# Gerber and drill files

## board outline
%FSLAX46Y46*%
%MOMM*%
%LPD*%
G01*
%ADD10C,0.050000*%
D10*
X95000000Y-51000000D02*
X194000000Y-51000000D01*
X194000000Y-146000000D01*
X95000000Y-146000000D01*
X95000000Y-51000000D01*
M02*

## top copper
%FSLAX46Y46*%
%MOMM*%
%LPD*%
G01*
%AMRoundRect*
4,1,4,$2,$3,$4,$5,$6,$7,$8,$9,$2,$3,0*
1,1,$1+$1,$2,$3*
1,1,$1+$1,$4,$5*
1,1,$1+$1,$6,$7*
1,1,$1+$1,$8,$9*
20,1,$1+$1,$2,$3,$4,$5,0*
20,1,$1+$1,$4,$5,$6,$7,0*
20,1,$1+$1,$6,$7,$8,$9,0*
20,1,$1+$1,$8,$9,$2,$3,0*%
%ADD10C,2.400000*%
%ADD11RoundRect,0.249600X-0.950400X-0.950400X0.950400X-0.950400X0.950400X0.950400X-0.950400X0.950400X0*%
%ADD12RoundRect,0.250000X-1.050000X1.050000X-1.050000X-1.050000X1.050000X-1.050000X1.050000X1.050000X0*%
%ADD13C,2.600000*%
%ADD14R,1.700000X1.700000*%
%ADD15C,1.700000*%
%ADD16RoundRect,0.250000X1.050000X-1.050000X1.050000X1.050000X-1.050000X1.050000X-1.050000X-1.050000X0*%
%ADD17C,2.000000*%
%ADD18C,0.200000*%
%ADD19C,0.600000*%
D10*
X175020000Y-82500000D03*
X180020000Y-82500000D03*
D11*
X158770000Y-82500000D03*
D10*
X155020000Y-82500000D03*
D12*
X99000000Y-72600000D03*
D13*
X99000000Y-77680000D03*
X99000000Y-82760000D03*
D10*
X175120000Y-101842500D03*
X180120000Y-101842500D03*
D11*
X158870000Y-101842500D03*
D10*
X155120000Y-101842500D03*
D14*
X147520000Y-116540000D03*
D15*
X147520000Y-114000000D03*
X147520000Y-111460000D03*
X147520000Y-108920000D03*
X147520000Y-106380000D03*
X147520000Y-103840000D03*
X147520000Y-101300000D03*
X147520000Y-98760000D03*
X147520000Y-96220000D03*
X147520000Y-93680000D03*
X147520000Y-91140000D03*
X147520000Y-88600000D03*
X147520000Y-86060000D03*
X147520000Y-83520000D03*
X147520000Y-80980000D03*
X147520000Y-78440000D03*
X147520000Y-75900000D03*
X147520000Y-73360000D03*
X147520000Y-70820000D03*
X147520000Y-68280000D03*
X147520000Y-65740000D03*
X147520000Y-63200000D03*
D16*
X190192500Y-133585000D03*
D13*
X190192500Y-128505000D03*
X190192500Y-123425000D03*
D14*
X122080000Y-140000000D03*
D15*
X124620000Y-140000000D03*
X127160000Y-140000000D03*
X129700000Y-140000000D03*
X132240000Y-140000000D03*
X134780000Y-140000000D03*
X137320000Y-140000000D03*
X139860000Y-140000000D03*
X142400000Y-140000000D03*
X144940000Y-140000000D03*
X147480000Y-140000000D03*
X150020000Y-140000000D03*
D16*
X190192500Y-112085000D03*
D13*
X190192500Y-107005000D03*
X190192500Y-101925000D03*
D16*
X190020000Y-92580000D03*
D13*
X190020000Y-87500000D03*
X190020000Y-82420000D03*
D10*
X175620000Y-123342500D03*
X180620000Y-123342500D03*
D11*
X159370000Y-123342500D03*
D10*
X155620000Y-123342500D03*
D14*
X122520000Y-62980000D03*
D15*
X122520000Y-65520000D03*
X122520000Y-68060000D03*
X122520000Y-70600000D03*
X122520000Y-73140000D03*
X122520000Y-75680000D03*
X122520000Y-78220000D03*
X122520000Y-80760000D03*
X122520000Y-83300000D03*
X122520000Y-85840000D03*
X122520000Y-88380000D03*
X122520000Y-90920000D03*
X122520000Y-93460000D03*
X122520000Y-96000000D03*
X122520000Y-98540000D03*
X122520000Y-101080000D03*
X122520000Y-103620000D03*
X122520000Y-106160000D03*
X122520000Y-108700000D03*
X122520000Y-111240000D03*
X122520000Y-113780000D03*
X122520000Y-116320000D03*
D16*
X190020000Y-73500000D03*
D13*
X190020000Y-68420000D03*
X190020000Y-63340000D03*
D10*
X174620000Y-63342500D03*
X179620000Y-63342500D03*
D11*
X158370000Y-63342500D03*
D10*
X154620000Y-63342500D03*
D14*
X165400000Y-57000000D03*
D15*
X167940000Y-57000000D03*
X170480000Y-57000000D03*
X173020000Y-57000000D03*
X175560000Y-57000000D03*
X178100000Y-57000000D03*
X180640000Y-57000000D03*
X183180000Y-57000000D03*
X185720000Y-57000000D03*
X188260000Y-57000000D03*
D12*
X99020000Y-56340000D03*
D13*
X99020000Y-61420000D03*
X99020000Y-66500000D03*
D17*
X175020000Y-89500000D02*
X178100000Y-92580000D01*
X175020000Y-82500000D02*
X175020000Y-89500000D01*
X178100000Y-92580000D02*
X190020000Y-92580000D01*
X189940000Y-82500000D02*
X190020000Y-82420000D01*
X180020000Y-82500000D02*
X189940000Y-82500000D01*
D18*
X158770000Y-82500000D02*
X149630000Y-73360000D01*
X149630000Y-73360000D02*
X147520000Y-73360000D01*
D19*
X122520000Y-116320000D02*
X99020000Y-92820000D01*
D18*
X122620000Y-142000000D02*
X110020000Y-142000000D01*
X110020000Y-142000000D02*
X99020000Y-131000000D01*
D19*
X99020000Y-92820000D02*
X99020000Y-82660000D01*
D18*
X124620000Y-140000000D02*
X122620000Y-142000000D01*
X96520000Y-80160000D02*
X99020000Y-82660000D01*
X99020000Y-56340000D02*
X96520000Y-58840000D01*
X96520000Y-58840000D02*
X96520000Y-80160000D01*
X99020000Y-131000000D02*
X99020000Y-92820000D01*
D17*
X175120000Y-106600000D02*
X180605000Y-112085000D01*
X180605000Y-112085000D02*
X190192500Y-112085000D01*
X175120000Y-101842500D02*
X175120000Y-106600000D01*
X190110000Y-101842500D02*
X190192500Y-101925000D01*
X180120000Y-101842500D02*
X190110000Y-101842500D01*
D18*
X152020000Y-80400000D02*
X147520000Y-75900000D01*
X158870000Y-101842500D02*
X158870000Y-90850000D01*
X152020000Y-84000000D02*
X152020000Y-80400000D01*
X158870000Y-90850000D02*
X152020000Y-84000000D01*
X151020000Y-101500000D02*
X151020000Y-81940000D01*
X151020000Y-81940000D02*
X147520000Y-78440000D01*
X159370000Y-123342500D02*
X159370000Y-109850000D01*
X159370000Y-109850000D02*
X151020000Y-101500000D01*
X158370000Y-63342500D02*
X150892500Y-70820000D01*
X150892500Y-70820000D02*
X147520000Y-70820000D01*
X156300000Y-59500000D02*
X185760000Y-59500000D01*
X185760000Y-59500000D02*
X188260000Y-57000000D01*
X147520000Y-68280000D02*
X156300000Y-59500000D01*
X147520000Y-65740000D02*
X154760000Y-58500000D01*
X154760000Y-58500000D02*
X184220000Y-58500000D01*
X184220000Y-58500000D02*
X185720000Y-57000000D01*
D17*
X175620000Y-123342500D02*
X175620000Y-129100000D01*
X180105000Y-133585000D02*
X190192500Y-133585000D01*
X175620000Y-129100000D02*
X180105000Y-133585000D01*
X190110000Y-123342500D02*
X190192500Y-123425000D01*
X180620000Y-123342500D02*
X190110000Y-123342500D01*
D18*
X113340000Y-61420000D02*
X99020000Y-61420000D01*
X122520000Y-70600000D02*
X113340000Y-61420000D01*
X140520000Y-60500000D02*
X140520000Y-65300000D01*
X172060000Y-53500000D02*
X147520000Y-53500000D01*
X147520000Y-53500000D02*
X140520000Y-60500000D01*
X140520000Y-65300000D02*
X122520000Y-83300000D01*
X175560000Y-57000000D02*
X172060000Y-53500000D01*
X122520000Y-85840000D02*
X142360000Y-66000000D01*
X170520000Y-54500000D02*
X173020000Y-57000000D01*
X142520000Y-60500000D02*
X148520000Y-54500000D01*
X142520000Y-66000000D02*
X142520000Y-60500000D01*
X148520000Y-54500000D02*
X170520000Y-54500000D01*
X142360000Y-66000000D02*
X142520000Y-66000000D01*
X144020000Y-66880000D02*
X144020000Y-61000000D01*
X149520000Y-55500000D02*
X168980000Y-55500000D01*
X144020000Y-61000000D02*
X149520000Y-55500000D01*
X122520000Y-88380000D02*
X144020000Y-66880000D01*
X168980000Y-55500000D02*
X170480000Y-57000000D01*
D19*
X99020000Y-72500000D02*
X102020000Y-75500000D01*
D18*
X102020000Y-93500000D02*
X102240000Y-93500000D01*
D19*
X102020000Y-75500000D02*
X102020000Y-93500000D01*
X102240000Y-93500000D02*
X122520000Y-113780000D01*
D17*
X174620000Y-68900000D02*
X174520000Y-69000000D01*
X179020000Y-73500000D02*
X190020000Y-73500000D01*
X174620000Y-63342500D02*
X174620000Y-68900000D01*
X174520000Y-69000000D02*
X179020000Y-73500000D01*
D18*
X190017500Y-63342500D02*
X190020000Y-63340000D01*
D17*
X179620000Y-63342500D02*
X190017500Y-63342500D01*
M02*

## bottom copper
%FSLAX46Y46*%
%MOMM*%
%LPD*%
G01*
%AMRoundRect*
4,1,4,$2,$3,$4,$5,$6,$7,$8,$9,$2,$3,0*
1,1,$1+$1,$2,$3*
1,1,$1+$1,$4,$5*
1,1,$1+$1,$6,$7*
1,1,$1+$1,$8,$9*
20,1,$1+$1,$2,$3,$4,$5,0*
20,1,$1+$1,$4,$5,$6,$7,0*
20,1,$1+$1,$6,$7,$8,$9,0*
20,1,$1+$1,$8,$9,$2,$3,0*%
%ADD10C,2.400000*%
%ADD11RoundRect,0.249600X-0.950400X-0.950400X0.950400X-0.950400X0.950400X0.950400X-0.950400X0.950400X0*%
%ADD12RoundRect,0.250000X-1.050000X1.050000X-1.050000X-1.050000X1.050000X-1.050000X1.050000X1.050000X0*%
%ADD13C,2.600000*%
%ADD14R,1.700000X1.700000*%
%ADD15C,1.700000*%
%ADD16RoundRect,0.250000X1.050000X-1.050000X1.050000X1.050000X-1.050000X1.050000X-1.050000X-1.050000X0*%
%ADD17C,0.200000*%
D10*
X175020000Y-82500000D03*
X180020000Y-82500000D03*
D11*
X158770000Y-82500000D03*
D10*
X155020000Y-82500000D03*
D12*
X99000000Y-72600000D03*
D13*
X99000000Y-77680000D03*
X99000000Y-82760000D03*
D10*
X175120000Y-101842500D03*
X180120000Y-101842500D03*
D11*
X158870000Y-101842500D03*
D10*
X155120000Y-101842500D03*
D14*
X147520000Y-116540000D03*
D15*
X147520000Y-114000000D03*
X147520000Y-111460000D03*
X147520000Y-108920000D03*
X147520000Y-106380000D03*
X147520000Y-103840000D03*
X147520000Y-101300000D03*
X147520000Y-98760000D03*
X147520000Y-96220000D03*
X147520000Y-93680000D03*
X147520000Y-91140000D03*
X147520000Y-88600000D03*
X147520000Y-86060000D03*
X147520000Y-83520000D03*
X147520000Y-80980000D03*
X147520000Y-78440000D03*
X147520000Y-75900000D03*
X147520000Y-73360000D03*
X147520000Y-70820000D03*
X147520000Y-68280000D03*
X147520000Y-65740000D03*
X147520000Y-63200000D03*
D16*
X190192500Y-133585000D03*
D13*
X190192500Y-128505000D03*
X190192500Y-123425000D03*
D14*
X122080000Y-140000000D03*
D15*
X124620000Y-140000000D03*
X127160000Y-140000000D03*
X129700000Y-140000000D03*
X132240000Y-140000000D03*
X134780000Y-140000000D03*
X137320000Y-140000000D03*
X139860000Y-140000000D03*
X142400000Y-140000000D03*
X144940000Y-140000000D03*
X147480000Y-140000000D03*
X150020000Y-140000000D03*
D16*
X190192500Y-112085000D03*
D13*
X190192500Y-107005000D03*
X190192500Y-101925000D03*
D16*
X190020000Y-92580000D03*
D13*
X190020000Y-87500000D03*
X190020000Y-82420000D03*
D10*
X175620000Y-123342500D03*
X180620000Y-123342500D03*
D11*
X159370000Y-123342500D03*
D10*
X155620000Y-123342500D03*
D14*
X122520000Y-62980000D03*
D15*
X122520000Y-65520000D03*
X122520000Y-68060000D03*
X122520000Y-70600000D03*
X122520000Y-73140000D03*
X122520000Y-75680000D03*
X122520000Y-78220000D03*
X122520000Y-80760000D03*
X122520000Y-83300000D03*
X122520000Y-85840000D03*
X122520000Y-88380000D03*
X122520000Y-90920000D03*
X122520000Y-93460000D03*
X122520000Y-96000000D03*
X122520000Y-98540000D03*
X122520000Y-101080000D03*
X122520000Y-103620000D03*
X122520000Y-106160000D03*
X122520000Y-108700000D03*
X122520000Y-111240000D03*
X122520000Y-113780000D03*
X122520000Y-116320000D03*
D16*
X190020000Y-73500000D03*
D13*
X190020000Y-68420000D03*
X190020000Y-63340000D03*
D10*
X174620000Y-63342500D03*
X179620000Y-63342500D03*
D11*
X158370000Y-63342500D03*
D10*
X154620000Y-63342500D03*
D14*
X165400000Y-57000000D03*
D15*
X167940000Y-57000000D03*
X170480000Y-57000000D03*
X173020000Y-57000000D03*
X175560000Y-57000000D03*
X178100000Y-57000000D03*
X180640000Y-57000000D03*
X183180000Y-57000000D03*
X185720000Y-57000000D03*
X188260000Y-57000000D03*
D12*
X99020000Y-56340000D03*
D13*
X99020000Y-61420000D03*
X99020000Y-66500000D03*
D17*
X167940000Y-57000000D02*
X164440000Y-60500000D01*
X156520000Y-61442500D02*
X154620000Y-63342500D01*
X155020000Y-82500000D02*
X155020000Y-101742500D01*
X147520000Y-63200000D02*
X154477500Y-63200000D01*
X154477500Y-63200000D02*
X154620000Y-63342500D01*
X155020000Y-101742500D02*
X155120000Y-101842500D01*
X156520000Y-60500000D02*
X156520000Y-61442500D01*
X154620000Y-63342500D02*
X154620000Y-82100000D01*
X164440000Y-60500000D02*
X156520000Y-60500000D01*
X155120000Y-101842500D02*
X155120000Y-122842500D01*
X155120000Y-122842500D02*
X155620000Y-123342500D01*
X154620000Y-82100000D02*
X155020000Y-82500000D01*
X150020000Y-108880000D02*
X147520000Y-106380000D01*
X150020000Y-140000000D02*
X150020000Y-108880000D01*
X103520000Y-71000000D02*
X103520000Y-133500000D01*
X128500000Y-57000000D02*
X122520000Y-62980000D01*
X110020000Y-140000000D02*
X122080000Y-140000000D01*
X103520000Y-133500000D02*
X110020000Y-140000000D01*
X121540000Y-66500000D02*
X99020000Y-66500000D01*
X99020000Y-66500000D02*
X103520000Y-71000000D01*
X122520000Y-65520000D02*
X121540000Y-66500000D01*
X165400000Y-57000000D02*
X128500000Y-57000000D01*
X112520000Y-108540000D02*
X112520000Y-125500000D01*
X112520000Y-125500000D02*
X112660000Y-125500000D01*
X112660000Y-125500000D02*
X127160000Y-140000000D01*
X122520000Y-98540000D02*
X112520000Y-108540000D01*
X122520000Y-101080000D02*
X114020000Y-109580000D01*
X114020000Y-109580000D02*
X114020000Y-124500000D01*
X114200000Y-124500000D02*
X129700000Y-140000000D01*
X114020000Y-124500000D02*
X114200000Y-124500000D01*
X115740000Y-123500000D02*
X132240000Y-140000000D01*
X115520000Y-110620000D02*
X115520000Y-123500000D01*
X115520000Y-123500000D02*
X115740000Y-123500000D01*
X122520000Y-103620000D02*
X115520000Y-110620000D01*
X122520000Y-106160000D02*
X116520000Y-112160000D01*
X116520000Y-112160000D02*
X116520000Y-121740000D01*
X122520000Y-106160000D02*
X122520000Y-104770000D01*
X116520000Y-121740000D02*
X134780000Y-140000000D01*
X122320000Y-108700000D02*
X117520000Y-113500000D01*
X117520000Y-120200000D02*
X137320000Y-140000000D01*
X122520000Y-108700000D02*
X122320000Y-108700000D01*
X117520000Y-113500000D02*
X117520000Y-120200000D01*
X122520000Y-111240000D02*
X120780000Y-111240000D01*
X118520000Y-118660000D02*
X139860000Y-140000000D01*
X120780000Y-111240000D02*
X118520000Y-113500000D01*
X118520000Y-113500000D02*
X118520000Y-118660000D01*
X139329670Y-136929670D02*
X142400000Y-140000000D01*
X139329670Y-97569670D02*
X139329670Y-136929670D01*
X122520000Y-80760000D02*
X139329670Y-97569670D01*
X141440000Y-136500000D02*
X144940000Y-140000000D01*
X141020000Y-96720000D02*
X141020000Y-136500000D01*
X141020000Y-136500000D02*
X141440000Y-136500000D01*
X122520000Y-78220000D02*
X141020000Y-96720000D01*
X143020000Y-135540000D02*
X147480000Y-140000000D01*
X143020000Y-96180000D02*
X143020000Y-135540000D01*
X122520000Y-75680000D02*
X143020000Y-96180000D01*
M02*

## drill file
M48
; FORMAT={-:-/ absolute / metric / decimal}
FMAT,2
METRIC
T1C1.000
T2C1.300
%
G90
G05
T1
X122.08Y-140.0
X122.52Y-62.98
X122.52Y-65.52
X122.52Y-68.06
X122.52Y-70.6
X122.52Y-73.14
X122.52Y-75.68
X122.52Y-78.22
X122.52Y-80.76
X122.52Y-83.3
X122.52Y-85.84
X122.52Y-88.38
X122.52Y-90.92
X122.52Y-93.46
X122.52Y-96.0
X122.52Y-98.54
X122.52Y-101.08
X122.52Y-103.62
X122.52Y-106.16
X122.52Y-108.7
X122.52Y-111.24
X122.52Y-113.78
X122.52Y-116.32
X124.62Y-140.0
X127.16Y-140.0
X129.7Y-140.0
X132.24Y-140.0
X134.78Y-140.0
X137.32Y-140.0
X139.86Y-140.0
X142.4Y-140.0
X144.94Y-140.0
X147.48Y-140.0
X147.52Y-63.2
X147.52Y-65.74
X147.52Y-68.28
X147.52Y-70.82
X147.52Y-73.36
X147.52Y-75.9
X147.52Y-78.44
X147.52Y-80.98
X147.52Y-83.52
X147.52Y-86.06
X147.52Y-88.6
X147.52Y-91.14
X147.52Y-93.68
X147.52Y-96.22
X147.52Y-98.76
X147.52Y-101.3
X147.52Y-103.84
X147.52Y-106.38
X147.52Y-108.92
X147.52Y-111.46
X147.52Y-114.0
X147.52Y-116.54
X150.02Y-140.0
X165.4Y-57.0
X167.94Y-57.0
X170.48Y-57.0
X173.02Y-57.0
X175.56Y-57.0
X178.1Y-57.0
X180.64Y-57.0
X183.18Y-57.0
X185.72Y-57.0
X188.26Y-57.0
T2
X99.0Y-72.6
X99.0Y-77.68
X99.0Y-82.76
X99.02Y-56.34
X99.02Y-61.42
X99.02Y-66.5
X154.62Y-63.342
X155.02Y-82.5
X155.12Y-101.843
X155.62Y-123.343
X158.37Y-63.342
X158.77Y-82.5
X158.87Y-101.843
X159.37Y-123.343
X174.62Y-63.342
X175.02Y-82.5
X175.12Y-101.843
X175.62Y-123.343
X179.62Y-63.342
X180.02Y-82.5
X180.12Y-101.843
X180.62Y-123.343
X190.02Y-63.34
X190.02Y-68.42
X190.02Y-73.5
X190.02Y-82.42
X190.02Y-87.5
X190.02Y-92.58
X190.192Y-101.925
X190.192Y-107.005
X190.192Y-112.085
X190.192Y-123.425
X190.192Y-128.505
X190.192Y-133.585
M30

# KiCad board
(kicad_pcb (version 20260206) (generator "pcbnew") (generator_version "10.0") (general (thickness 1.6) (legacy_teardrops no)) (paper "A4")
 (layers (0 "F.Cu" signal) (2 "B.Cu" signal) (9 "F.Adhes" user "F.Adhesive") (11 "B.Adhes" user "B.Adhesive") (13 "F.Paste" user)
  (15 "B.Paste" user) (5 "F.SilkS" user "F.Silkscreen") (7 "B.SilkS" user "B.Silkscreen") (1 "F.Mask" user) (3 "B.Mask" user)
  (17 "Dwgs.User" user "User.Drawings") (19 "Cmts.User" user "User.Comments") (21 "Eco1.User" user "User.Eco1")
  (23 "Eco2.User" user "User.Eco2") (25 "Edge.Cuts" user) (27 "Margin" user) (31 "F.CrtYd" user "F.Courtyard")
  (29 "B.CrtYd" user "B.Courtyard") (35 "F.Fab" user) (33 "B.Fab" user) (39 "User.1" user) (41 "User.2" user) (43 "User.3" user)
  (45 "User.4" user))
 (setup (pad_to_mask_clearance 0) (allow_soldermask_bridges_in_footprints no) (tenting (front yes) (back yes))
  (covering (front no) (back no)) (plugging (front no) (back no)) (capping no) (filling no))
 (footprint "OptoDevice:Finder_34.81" (layer "F.Cu") (at 158.77 82.5)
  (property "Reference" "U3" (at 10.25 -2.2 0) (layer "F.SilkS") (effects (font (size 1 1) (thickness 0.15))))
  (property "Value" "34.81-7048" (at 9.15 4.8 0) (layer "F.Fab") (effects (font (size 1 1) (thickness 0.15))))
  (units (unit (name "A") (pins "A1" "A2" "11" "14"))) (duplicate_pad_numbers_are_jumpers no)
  (pad "11" thru_hole circle (at 16.25 0) (size 2.4 2.4) (drill 1.3) (layers "*.Cu" "*.Mask") (remove_unused_layers no)
   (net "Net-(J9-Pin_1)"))
  (pad "14" thru_hole circle (at 21.25 0) (size 2.4 2.4) (drill 1.3) (layers "*.Cu" "*.Mask") (remove_unused_layers no)
   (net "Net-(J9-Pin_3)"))
  (pad "A1" thru_hole roundrect (at 0 0) (size 2.4 2.4) (drill 1.3) (layers "*.Cu" "*.Mask") (remove_unused_layers no)
   (roundrect_rratio 0.104) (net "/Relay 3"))
  (pad "A2" thru_hole circle (at -3.75 0) (size 2.4 2.4) (drill 1.3) (layers "*.Cu" "*.Mask") (remove_unused_layers no) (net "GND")))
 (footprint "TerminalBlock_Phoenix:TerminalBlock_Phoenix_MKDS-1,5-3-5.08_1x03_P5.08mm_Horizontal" (layer "F.Cu") (at 99 72.6 -90)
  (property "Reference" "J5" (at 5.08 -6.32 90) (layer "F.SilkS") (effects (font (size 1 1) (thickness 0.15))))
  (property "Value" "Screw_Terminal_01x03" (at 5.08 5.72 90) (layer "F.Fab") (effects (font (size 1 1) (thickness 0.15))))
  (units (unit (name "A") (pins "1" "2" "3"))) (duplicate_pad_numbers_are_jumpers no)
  (pad "1" thru_hole roundrect (at 0 0 270) (size 2.6 2.6) (drill 1.3) (layers "*.Cu" "*.Mask") (remove_unused_layers no)
   (roundrect_rratio 0.096154) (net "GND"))
  (pad "2" thru_hole circle (at 5.08 0 270) (size 2.6 2.6) (drill 1.3) (layers "*.Cu" "*.Mask") (remove_unused_layers no)
   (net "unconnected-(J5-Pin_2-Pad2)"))
  (pad "3" thru_hole circle (at 10.16 0 270) (size 2.6 2.6) (drill 1.3) (layers "*.Cu" "*.Mask") (remove_unused_layers no) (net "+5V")))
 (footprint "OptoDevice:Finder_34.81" (layer "F.Cu") (at 158.87 101.8425)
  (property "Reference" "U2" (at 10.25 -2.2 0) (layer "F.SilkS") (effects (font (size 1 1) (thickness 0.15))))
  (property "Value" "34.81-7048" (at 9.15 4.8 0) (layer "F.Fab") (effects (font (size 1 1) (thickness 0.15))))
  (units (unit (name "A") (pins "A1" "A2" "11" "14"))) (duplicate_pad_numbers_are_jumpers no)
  (pad "11" thru_hole circle (at 16.25 0) (size 2.4 2.4) (drill 1.3) (layers "*.Cu" "*.Mask") (remove_unused_layers no)
   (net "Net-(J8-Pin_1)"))
  (pad "14" thru_hole circle (at 21.25 0) (size 2.4 2.4) (drill 1.3) (layers "*.Cu" "*.Mask") (remove_unused_layers no)
   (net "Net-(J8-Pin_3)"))
  (pad "A1" thru_hole roundrect (at 0 0) (size 2.4 2.4) (drill 1.3) (layers "*.Cu" "*.Mask") (remove_unused_layers no)
   (roundrect_rratio 0.104) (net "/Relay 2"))
  (pad "A2" thru_hole circle (at -3.75 0) (size 2.4 2.4) (drill 1.3) (layers "*.Cu" "*.Mask") (remove_unused_layers no) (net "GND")))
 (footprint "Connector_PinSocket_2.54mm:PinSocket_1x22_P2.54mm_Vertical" (layer "F.Cu") (at 147.52 116.54 180)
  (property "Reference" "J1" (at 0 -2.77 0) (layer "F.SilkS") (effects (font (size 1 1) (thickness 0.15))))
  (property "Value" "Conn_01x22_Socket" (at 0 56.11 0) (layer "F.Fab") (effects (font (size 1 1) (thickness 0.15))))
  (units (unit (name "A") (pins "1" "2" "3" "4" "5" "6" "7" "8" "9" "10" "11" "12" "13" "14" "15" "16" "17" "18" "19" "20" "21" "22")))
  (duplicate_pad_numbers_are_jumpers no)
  (pad "1" thru_hole rect (at 0 0 180) (size 1.7 1.7) (drill 1) (layers "*.Cu" "*.Mask") (remove_unused_layers no) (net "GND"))
  (pad "2" thru_hole circle (at 0 2.54 180) (size 1.7 1.7) (drill 1) (layers "*.Cu" "*.Mask") (remove_unused_layers no) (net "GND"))
  (pad "3" thru_hole circle (at 0 5.08 180) (size 1.7 1.7) (drill 1) (layers "*.Cu" "*.Mask") (remove_unused_layers no)
   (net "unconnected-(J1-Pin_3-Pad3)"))
  (pad "4" thru_hole circle (at 0 7.62 180) (size 1.7 1.7) (drill 1) (layers "*.Cu" "*.Mask") (remove_unused_layers no)
   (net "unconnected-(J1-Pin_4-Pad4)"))
  (pad "5" thru_hole circle (at 0 10.16 180) (size 1.7 1.7) (drill 1) (layers "*.Cu" "*.Mask") (remove_unused_layers no) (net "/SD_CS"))
  (pad "6" thru_hole circle (at 0 12.7 180) (size 1.7 1.7) (drill 1) (layers "*.Cu" "*.Mask") (remove_unused_layers no)
   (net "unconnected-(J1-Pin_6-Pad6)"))
  (pad "7" thru_hole circle (at 0 15.24 180) (size 1.7 1.7) (drill 1) (layers "*.Cu" "*.Mask") (remove_unused_layers no)
   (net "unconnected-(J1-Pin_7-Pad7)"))
  (pad "8" thru_hole circle (at 0 17.78 180) (size 1.7 1.7) (drill 1) (layers "*.Cu" "*.Mask") (remove_unused_layers no)
   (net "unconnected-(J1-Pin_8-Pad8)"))
  (pad "9" thru_hole circle (at 0 20.32 180) (size 1.7 1.7) (drill 1) (layers "*.Cu" "*.Mask") (remove_unused_layers no)
   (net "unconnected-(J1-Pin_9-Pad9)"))
  (pad "10" thru_hole circle (at 0 22.86 180) (size 1.7 1.7) (drill 1) (layers "*.Cu" "*.Mask") (remove_unused_layers no)
   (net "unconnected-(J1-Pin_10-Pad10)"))
  (pad "11" thru_hole circle (at 0 25.4 180) (size 1.7 1.7) (drill 1) (layers "*.Cu" "*.Mask") (remove_unused_layers no)
   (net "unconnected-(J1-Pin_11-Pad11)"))
  (pad "12" thru_hole circle (at 0 27.94 180) (size 1.7 1.7) (drill 1) (layers "*.Cu" "*.Mask") (remove_unused_layers no)
   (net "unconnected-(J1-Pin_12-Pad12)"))
  (pad "13" thru_hole circle (at 0 30.48 180) (size 1.7 1.7) (drill 1) (layers "*.Cu" "*.Mask") (remove_unused_layers no)
   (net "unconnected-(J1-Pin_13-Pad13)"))
  (pad "14" thru_hole circle (at 0 33.02 180) (size 1.7 1.7) (drill 1) (layers "*.Cu" "*.Mask") (remove_unused_layers no)
   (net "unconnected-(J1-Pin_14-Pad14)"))
  (pad "15" thru_hole circle (at 0 35.56 180) (size 1.7 1.7) (drill 1) (layers "*.Cu" "*.Mask") (remove_unused_layers no)
   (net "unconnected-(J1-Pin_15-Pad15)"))
  (pad "16" thru_hole circle (at 0 38.1 180) (size 1.7 1.7) (drill 1) (layers "*.Cu" "*.Mask") (remove_unused_layers no) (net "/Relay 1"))
  (pad "17" thru_hole circle (at 0 40.64 180) (size 1.7 1.7) (drill 1) (layers "*.Cu" "*.Mask") (remove_unused_layers no) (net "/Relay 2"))
  (pad "18" thru_hole circle (at 0 43.18 180) (size 1.7 1.7) (drill 1) (layers "*.Cu" "*.Mask") (remove_unused_layers no) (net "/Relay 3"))
  (pad "19" thru_hole circle (at 0 45.72 180) (size 1.7 1.7) (drill 1) (layers "*.Cu" "*.Mask") (remove_unused_layers no) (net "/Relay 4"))
  (pad "20" thru_hole circle (at 0 48.26 180) (size 1.7 1.7) (drill 1) (layers "*.Cu" "*.Mask") (remove_unused_layers no) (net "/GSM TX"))
  (pad "21" thru_hole circle (at 0 50.8 180) (size 1.7 1.7) (drill 1) (layers "*.Cu" "*.Mask") (remove_unused_layers no) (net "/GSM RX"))
  (pad "22" thru_hole circle (at 0 53.34 180) (size 1.7 1.7) (drill 1) (layers "*.Cu" "*.Mask") (remove_unused_layers no) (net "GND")))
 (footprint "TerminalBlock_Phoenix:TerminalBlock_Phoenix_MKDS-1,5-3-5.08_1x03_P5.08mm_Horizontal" (layer "F.Cu") (at 190.1925 133.585 90)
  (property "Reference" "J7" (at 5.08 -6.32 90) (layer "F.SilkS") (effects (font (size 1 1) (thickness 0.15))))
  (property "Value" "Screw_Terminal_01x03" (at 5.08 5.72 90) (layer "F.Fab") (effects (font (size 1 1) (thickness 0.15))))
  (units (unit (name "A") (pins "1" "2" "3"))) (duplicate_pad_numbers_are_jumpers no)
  (pad "1" thru_hole roundrect (at 0 0 90) (size 2.6 2.6) (drill 1.3) (layers "*.Cu" "*.Mask") (remove_unused_layers no)
   (roundrect_rratio 0.096154) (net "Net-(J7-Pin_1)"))
  (pad "2" thru_hole circle (at 5.08 0 90) (size 2.6 2.6) (drill 1.3) (layers "*.Cu" "*.Mask") (remove_unused_layers no)
   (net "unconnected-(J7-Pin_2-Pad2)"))
  (pad "3" thru_hole circle (at 10.16 0 90) (size 2.6 2.6) (drill 1.3) (layers "*.Cu" "*.Mask") (remove_unused_layers no)
   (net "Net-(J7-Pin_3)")))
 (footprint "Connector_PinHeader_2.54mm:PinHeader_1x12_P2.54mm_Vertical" (layer "F.Cu") (at 122.08 140 90)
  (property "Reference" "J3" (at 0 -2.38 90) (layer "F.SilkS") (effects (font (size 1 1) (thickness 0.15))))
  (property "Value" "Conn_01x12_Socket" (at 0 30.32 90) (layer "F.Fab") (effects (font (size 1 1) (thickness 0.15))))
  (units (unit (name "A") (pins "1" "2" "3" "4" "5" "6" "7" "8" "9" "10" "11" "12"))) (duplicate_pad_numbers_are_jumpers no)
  (pad "1" thru_hole rect (at 0 0 90) (size 1.7 1.7) (drill 1) (layers "*.Cu" "*.Mask") (remove_unused_layers no) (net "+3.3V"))
  (pad "2" thru_hole circle (at 0 2.54 90) (size 1.7 1.7) (drill 1) (layers "*.Cu" "*.Mask") (remove_unused_layers no) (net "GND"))
  (pad "3" thru_hole circle (at 0 5.08 90) (size 1.7 1.7) (drill 1) (layers "*.Cu" "*.Mask") (remove_unused_layers no) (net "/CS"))
  (pad "4" thru_hole circle (at 0 7.62 90) (size 1.7 1.7) (drill 1) (layers "*.Cu" "*.Mask") (remove_unused_layers no) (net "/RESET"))
  (pad "5" thru_hole circle (at 0 10.16 90) (size 1.7 1.7) (drill 1) (layers "*.Cu" "*.Mask") (remove_unused_layers no) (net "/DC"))
  (pad "6" thru_hole circle (at 0 12.7 90) (size 1.7 1.7) (drill 1) (layers "*.Cu" "*.Mask") (remove_unused_layers no) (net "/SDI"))
  (pad "7" thru_hole circle (at 0 15.24 90) (size 1.7 1.7) (drill 1) (layers "*.Cu" "*.Mask") (remove_unused_layers no) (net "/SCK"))
  (pad "8" thru_hole circle (at 0 17.78 90) (size 1.7 1.7) (drill 1) (layers "*.Cu" "*.Mask") (remove_unused_layers no) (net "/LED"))
  (pad "9" thru_hole circle (at 0 20.32 90) (size 1.7 1.7) (drill 1) (layers "*.Cu" "*.Mask") (remove_unused_layers no) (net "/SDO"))
  (pad "10" thru_hole circle (at 0 22.86 90) (size 1.7 1.7) (drill 1) (layers "*.Cu" "*.Mask") (remove_unused_layers no) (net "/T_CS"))
  (pad "11" thru_hole circle (at 0 25.4 90) (size 1.7 1.7) (drill 1) (layers "*.Cu" "*.Mask") (remove_unused_layers no) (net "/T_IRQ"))
  (pad "12" thru_hole circle (at 0 27.94 90) (size 1.7 1.7) (drill 1) (layers "*.Cu" "*.Mask") (remove_unused_layers no) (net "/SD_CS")))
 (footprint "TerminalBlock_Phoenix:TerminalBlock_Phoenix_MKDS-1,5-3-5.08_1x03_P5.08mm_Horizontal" (layer "F.Cu") (at 190.1925 112.085 90)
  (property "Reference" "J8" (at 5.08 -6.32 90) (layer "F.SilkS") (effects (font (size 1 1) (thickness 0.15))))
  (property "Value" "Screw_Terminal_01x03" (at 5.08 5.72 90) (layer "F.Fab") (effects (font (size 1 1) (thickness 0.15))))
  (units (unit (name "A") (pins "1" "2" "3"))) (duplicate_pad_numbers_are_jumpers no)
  (pad "1" thru_hole roundrect (at 0 0 90) (size 2.6 2.6) (drill 1.3) (layers "*.Cu" "*.Mask") (remove_unused_layers no)
   (roundrect_rratio 0.096154) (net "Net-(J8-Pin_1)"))
  (pad "2" thru_hole circle (at 5.08 0 90) (size 2.6 2.6) (drill 1.3) (layers "*.Cu" "*.Mask") (remove_unused_layers no)
   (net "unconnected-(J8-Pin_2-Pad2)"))
  (pad "3" thru_hole circle (at 10.16 0 90) (size 2.6 2.6) (drill 1.3) (layers "*.Cu" "*.Mask") (remove_unused_layers no)
   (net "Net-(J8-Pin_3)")))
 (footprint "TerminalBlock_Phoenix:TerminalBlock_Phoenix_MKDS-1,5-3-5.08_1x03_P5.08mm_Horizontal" (layer "F.Cu") (at 190.02 92.58 90)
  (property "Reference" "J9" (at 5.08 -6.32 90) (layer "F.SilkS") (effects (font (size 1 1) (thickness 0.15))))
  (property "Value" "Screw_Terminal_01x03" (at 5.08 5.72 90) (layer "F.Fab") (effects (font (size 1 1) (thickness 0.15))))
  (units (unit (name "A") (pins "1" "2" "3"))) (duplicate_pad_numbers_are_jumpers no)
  (pad "1" thru_hole roundrect (at 0 0 90) (size 2.6 2.6) (drill 1.3) (layers "*.Cu" "*.Mask") (remove_unused_layers no)
   (roundrect_rratio 0.096154) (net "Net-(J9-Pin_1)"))
  (pad "2" thru_hole circle (at 5.08 0 90) (size 2.6 2.6) (drill 1.3) (layers "*.Cu" "*.Mask") (remove_unused_layers no)
   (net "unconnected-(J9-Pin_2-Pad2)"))
  (pad "3" thru_hole circle (at 10.16 0 90) (size 2.6 2.6) (drill 1.3) (layers "*.Cu" "*.Mask") (remove_unused_layers no)
   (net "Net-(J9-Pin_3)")))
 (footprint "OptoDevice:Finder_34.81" (layer "F.Cu") (at 159.37 123.3425)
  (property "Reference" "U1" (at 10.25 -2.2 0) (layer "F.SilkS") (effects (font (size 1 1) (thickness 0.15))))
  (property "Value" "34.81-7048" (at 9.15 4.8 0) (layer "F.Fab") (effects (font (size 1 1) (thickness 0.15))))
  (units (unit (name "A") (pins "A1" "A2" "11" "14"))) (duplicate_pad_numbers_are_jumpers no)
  (pad "11" thru_hole circle (at 16.25 0) (size 2.4 2.4) (drill 1.3) (layers "*.Cu" "*.Mask") (remove_unused_layers no)
   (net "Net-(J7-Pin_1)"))
  (pad "14" thru_hole circle (at 21.25 0) (size 2.4 2.4) (drill 1.3) (layers "*.Cu" "*.Mask") (remove_unused_layers no)
   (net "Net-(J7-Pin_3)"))
  (pad "A1" thru_hole roundrect (at 0 0) (size 2.4 2.4) (drill 1.3) (layers "*.Cu" "*.Mask") (remove_unused_layers no)
   (roundrect_rratio 0.104) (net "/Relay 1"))
  (pad "A2" thru_hole circle (at -3.75 0) (size 2.4 2.4) (drill 1.3) (layers "*.Cu" "*.Mask") (remove_unused_layers no) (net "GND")))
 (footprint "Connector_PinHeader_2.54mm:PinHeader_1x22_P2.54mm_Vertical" (layer "F.Cu") (at 122.52 62.98)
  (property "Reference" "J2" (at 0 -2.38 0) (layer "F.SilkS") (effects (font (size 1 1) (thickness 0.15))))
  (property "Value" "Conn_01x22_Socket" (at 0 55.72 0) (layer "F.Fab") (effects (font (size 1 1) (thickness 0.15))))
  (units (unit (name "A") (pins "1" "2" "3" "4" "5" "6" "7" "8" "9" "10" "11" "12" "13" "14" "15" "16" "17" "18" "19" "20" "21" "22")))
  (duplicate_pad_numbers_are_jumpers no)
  (pad "1" thru_hole rect (at 0 0) (size 1.7 1.7) (drill 1) (layers "*.Cu" "*.Mask") (remove_unused_layers no) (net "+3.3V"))
  (pad "2" thru_hole circle (at 0 2.54) (size 1.7 1.7) (drill 1) (layers "*.Cu" "*.Mask") (remove_unused_layers no) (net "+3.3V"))
  (pad "3" thru_hole circle (at 0 5.08) (size 1.7 1.7) (drill 1) (layers "*.Cu" "*.Mask") (remove_unused_layers no)
   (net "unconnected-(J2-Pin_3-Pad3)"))
  (pad "4" thru_hole circle (at 0 7.62) (size 1.7 1.7) (drill 1) (layers "*.Cu" "*.Mask") (remove_unused_layers no)
   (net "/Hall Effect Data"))
  (pad "5" thru_hole circle (at 0 10.16) (size 1.7 1.7) (drill 1) (layers "*.Cu" "*.Mask") (remove_unused_layers no)
   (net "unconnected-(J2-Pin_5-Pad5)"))
  (pad "6" thru_hole circle (at 0 12.7) (size 1.7 1.7) (drill 1) (layers "*.Cu" "*.Mask") (remove_unused_layers no) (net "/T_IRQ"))
  (pad "7" thru_hole circle (at 0 15.24) (size 1.7 1.7) (drill 1) (layers "*.Cu" "*.Mask") (remove_unused_layers no) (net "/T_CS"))
  (pad "8" thru_hole circle (at 0 17.78) (size 1.7 1.7) (drill 1) (layers "*.Cu" "*.Mask") (remove_unused_layers no) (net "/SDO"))
  (pad "9" thru_hole circle (at 0 20.32) (size 1.7 1.7) (drill 1) (layers "*.Cu" "*.Mask") (remove_unused_layers no) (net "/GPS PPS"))
  (pad "10" thru_hole circle (at 0 22.86) (size 1.7 1.7) (drill 1) (layers "*.Cu" "*.Mask") (remove_unused_layers no) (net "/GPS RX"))
  (pad "11" thru_hole circle (at 0 25.4) (size 1.7 1.7) (drill 1) (layers "*.Cu" "*.Mask") (remove_unused_layers no) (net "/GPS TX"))
  (pad "12" thru_hole circle (at 0 27.94) (size 1.7 1.7) (drill 1) (layers "*.Cu" "*.Mask") (remove_unused_layers no)
   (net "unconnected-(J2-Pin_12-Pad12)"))
  (pad "13" thru_hole circle (at 0 30.48) (size 1.7 1.7) (drill 1) (layers "*.Cu" "*.Mask") (remove_unused_layers no)
   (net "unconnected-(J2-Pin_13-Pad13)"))
  (pad "14" thru_hole circle (at 0 33.02) (size 1.7 1.7) (drill 1) (layers "*.Cu" "*.Mask") (remove_unused_layers no)
   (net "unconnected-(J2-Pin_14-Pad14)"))
  (pad "15" thru_hole circle (at 0 35.56) (size 1.7 1.7) (drill 1) (layers "*.Cu" "*.Mask") (remove_unused_layers no) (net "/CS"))
  (pad "16" thru_hole circle (at 0 38.1) (size 1.7 1.7) (drill 1) (layers "*.Cu" "*.Mask") (remove_unused_layers no) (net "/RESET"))
  (pad "17" thru_hole circle (at 0 40.64) (size 1.7 1.7) (drill 1) (layers "*.Cu" "*.Mask") (remove_unused_layers no) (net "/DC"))
  (pad "18" thru_hole circle (at 0 43.18) (size 1.7 1.7) (drill 1) (layers "*.Cu" "*.Mask") (remove_unused_layers no) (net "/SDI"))
  (pad "19" thru_hole circle (at 0 45.72) (size 1.7 1.7) (drill 1) (layers "*.Cu" "*.Mask") (remove_unused_layers no) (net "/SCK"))
  (pad "20" thru_hole circle (at 0 48.26) (size 1.7 1.7) (drill 1) (layers "*.Cu" "*.Mask") (remove_unused_layers no) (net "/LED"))
  (pad "21" thru_hole circle (at 0 50.8) (size 1.7 1.7) (drill 1) (layers "*.Cu" "*.Mask") (remove_unused_layers no) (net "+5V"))
  (pad "22" thru_hole circle (at 0 53.34) (size 1.7 1.7) (drill 1) (layers "*.Cu" "*.Mask") (remove_unused_layers no) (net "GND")))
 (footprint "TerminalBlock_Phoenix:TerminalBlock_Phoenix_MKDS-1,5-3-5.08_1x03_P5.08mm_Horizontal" (layer "F.Cu") (at 190.02 73.5 90)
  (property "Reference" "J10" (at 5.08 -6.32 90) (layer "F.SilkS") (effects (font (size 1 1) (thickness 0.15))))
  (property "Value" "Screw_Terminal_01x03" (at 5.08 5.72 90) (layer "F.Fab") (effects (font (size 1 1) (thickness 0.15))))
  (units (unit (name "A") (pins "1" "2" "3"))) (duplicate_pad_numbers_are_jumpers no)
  (pad "1" thru_hole roundrect (at 0 0 90) (size 2.6 2.6) (drill 1.3) (layers "*.Cu" "*.Mask") (remove_unused_layers no)
   (roundrect_rratio 0.096154) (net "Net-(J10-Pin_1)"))
  (pad "2" thru_hole circle (at 5.08 0 90) (size 2.6 2.6) (drill 1.3) (layers "*.Cu" "*.Mask") (remove_unused_layers no)
   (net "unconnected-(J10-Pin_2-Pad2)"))
  (pad "3" thru_hole circle (at 10.16 0 90) (size 2.6 2.6) (drill 1.3) (layers "*.Cu" "*.Mask") (remove_unused_layers no)
   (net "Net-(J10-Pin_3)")))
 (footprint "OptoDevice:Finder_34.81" (layer "F.Cu") (at 158.37 63.3425)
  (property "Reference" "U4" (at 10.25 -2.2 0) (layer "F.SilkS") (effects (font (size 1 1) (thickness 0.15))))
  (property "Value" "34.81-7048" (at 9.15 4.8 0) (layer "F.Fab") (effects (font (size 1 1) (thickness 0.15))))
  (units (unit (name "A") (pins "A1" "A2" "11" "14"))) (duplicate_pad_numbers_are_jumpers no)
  (pad "11" thru_hole circle (at 16.25 0) (size 2.4 2.4) (drill 1.3) (layers "*.Cu" "*.Mask") (remove_unused_layers no)
   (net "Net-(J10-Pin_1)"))
  (pad "14" thru_hole circle (at 21.25 0) (size 2.4 2.4) (drill 1.3) (layers "*.Cu" "*.Mask") (remove_unused_layers no)
   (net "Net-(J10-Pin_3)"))
  (pad "A1" thru_hole roundrect (at 0 0) (size 2.4 2.4) (drill 1.3) (layers "*.Cu" "*.Mask") (remove_unused_layers no)
   (roundrect_rratio 0.104) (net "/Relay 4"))
  (pad "A2" thru_hole circle (at -3.75 0) (size 2.4 2.4) (drill 1.3) (layers "*.Cu" "*.Mask") (remove_unused_layers no) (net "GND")))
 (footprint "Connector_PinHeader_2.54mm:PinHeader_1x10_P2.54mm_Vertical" (layer "F.Cu") (at 165.4 57 90)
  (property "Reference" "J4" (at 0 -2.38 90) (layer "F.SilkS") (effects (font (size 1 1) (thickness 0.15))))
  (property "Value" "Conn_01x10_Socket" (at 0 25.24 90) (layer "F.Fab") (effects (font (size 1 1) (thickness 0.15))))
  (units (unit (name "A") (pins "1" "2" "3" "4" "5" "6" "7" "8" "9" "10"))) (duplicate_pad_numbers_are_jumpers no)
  (pad "1" thru_hole rect (at 0 0 90) (size 1.7 1.7) (drill 1) (layers "*.Cu" "*.Mask") (remove_unused_layers no) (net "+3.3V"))
  (pad "2" thru_hole circle (at 0 2.54 90) (size 1.7 1.7) (drill 1) (layers "*.Cu" "*.Mask") (remove_unused_layers no) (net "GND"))
  (pad "3" thru_hole circle (at 0 5.08 90) (size 1.7 1.7) (drill 1) (layers "*.Cu" "*.Mask") (remove_unused_layers no) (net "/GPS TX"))
  (pad "4" thru_hole circle (at 0 7.62 90) (size 1.7 1.7) (drill 1) (layers "*.Cu" "*.Mask") (remove_unused_layers no) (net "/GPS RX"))
  (pad "5" thru_hole circle (at 0 10.16 90) (size 1.7 1.7) (drill 1) (layers "*.Cu" "*.Mask") (remove_unused_layers no) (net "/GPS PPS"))
  (pad "6" thru_hole circle (at 0 12.7 90) (size 1.7 1.7) (drill 1) (layers "*.Cu" "*.Mask") (remove_unused_layers no)
   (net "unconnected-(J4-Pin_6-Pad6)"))
  (pad "7" thru_hole circle (at 0 15.24 90) (size 1.7 1.7) (drill 1) (layers "*.Cu" "*.Mask") (remove_unused_layers no)
   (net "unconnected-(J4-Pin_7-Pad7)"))
  (pad "8" thru_hole circle (at 0 17.78 90) (size 1.7 1.7) (drill 1) (layers "*.Cu" "*.Mask") (remove_unused_layers no)
   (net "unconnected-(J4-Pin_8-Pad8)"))
  (pad "9" thru_hole circle (at 0 20.32 90) (size 1.7 1.7) (drill 1) (layers "*.Cu" "*.Mask") (remove_unused_layers no) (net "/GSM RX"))
  (pad "10" thru_hole circle (at 0 22.86 90) (size 1.7 1.7) (drill 1) (layers "*.Cu" "*.Mask") (remove_unused_layers no) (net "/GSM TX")))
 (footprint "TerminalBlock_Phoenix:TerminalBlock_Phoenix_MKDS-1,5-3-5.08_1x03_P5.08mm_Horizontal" (layer "F.Cu") (at 99.02 56.34 -90)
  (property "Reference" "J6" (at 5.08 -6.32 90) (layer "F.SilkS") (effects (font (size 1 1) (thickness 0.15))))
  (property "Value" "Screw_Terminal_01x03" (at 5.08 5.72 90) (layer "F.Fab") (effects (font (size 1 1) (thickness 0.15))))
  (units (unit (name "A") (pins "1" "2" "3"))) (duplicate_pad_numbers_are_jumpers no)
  (pad "1" thru_hole roundrect (at 0 0 270) (size 2.6 2.6) (drill 1.3) (layers "*.Cu" "*.Mask") (remove_unused_layers no)
   (roundrect_rratio 0.096154) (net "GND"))
  (pad "2" thru_hole circle (at 5.08 0 270) (size 2.6 2.6) (drill 1.3) (layers "*.Cu" "*.Mask") (remove_unused_layers no)
   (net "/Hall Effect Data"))
  (pad "3" thru_hole circle (at 10.16 0 270) (size 2.6 2.6) (drill 1.3) (layers "*.Cu" "*.Mask") (remove_unused_layers no) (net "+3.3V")))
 (gr_rect (start 95 51) (end 194 146) (stroke (width 0.05) (type default)) (fill no) (layer "Edge.Cuts"))
 (segment (start 175.02 89.5) (end 178.1 92.58) (width 2) (layer "F.Cu") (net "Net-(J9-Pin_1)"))
 (segment (start 175.02 82.5) (end 175.02 89.5) (width 2) (layer "F.Cu") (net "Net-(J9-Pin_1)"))
 (segment (start 178.1 92.58) (end 190.02 92.58) (width 2) (layer "F.Cu") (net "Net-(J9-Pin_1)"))
 (segment (start 189.94 82.5) (end 190.02 82.42) (width 2) (layer "F.Cu") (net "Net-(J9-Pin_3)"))
 (segment (start 180.02 82.5) (end 189.94 82.5) (width 2) (layer "F.Cu") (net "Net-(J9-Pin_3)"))
 (segment (start 158.77 82.5) (end 149.63 73.36) (width 0.2) (layer "F.Cu") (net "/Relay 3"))
 (segment (start 149.63 73.36) (end 147.52 73.36) (width 0.2) (layer "F.Cu") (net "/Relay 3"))
 (segment (start 122.52 116.32) (end 99.02 92.82) (width 0.6) (layer "F.Cu") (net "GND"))
 (segment (start 122.62 142) (end 110.02 142) (width 0.2) (layer "F.Cu") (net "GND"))
 (segment (start 110.02 142) (end 99.02 131) (width 0.2) (layer "F.Cu") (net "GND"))
 (segment (start 99.02 92.82) (end 99.02 82.66) (width 0.6) (layer "F.Cu") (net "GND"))
 (segment (start 124.62 140) (end 122.62 142) (width 0.2) (layer "F.Cu") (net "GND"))
 (segment (start 96.52 80.16) (end 99.02 82.66) (width 0.2) (layer "F.Cu") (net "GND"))
 (segment (start 99.02 56.34) (end 96.52 58.84) (width 0.2) (layer "F.Cu") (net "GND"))
 (segment (start 96.52 58.84) (end 96.52 80.16) (width 0.2) (layer "F.Cu") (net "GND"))
 (segment (start 99.02 131) (end 99.02 92.82) (width 0.2) (layer "F.Cu") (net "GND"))
 (segment (start 167.94 57) (end 164.44 60.5) (width 0.2) (layer "B.Cu") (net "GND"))
 (segment (start 156.52 61.4425) (end 154.62 63.3425) (width 0.2) (layer "B.Cu") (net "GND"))
 (segment (start 155.02 82.5) (end 155.02 101.7425) (width 0.2) (layer "B.Cu") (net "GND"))
 (segment (start 147.52 63.2) (end 154.4775 63.2) (width 0.2) (layer "B.Cu") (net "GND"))
 (segment (start 154.4775 63.2) (end 154.62 63.3425) (width 0.2) (layer "B.Cu") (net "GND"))
 (segment (start 155.02 101.7425) (end 155.12 101.8425) (width 0.2) (layer "B.Cu") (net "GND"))
 (segment (start 156.52 60.5) (end 156.52 61.4425) (width 0.2) (layer "B.Cu") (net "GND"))
 (segment (start 154.62 63.3425) (end 154.62 82.1) (width 0.2) (layer "B.Cu") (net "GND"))
 (segment (start 164.44 60.5) (end 156.52 60.5) (width 0.2) (layer "B.Cu") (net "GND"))
 (segment (start 155.12 101.8425) (end 155.12 122.8425) (width 0.2) (layer "B.Cu") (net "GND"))
 (segment (start 155.12 122.8425) (end 155.62 123.3425) (width 0.2) (layer "B.Cu") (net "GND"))
 (segment (start 154.62 82.1) (end 155.02 82.5) (width 0.2) (layer "B.Cu") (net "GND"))
 (segment (start 175.12 106.6) (end 180.605 112.085) (width 2) (layer "F.Cu") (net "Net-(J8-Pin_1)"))
 (segment (start 180.605 112.085) (end 190.1925 112.085) (width 2) (layer "F.Cu") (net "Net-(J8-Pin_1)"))
 (segment (start 175.12 101.8425) (end 175.12 106.6) (width 2) (layer "F.Cu") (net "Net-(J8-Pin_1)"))
 (segment (start 190.11 101.8425) (end 190.1925 101.925) (width 2) (layer "F.Cu") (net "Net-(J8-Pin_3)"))
 (segment (start 180.12 101.8425) (end 190.11 101.8425) (width 2) (layer "F.Cu") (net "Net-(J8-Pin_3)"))
 (segment (start 152.02 80.4) (end 147.52 75.9) (width 0.2) (layer "F.Cu") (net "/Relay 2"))
 (segment (start 158.87 101.8425) (end 158.87 90.85) (width 0.2) (layer "F.Cu") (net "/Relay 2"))
 (segment (start 152.02 84) (end 152.02 80.4) (width 0.2) (layer "F.Cu") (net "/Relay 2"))
 (segment (start 158.87 90.85) (end 152.02 84) (width 0.2) (layer "F.Cu") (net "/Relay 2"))
 (segment (start 150.02 108.88) (end 147.52 106.38) (width 0.2) (layer "B.Cu") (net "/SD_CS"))
 (segment (start 150.02 140) (end 150.02 108.88) (width 0.2) (layer "B.Cu") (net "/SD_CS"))
 (segment (start 151.02 101.5) (end 151.02 81.94) (width 0.2) (layer "F.Cu") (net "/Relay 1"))
 (segment (start 151.02 81.94) (end 147.52 78.44) (width 0.2) (layer "F.Cu") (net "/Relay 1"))
 (segment (start 159.37 123.3425) (end 159.37 109.85) (width 0.2) (layer "F.Cu") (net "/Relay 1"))
 (segment (start 159.37 109.85) (end 151.02 101.5) (width 0.2) (layer "F.Cu") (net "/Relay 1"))
 (segment (start 158.37 63.3425) (end 150.8925 70.82) (width 0.2) (layer "F.Cu") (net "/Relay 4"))
 (segment (start 150.8925 70.82) (end 147.52 70.82) (width 0.2) (layer "F.Cu") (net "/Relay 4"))
 (segment (start 156.3 59.5) (end 185.76 59.5) (width 0.2) (layer "F.Cu") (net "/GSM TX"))
 (segment (start 185.76 59.5) (end 188.26 57) (width 0.2) (layer "F.Cu") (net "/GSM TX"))
 (segment (start 147.52 68.28) (end 156.3 59.5) (width 0.2) (layer "F.Cu") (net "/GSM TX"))
 (segment (start 147.52 65.74) (end 154.76 58.5) (width 0.2) (layer "F.Cu") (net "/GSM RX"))
 (segment (start 154.76 58.5) (end 184.22 58.5) (width 0.2) (layer "F.Cu") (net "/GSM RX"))
 (segment (start 184.22 58.5) (end 185.72 57) (width 0.2) (layer "F.Cu") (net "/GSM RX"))
 (segment (start 175.62 123.3425) (end 175.62 129.1) (width 2) (layer "F.Cu") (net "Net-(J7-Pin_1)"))
 (segment (start 180.105 133.585) (end 190.1925 133.585) (width 2) (layer "F.Cu") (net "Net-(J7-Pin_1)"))
 (segment (start 175.62 129.1) (end 180.105 133.585) (width 2) (layer "F.Cu") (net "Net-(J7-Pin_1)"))
 (segment (start 190.11 123.3425) (end 190.1925 123.425) (width 2) (layer "F.Cu") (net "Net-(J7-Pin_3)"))
 (segment (start 180.62 123.3425) (end 190.11 123.3425) (width 2) (layer "F.Cu") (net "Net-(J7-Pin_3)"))
 (segment (start 103.52 71) (end 103.52 133.5) (width 0.2) (layer "B.Cu") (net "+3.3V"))
 (segment (start 128.5 57) (end 122.52 62.98) (width 0.2) (layer "B.Cu") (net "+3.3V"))
 (segment (start 110.02 140) (end 122.08 140) (width 0.2) (layer "B.Cu") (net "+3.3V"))
 (segment (start 103.52 133.5) (end 110.02 140) (width 0.2) (layer "B.Cu") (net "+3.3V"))
 (segment (start 121.54 66.5) (end 99.02 66.5) (width 0.2) (layer "B.Cu") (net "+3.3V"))
 (segment (start 99.02 66.5) (end 103.52 71) (width 0.2) (layer "B.Cu") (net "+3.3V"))
 (segment (start 122.52 65.52) (end 121.54 66.5) (width 0.2) (layer "B.Cu") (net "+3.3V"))
 (segment (start 165.4 57) (end 128.5 57) (width 0.2) (layer "B.Cu") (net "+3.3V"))
 (segment (start 112.52 108.54) (end 112.52 125.5) (width 0.2) (layer "B.Cu") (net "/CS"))
 (segment (start 112.52 125.5) (end 112.66 125.5) (width 0.2) (layer "B.Cu") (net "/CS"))
 (segment (start 112.66 125.5) (end 127.16 140) (width 0.2) (layer "B.Cu") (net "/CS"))
 (segment (start 122.52 98.54) (end 112.52 108.54) (width 0.2) (layer "B.Cu") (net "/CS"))
 (segment (start 122.52 101.08) (end 114.02 109.58) (width 0.2) (layer "B.Cu") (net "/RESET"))
 (segment (start 114.02 109.58) (end 114.02 124.5) (width 0.2) (layer "B.Cu") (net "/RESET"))
 (segment (start 114.2 124.5) (end 129.7 140) (width 0.2) (layer "B.Cu") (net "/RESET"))
 (segment (start 114.02 124.5) (end 114.2 124.5) (width 0.2) (layer "B.Cu") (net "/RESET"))
 (segment (start 115.74 123.5) (end 132.24 140) (width 0.2) (layer "B.Cu") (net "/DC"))
 (segment (start 115.52 110.62) (end 115.52 123.5) (width 0.2) (layer "B.Cu") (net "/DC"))
 (segment (start 115.52 123.5) (end 115.74 123.5) (width 0.2) (layer "B.Cu") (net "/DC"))
 (segment (start 122.52 103.62) (end 115.52 110.62) (width 0.2) (layer "B.Cu") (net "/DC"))
 (segment (start 122.52 106.16) (end 116.52 112.16) (width 0.2) (layer "B.Cu") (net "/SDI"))
 (segment (start 116.52 112.16) (end 116.52 121.74) (width 0.2) (layer "B.Cu") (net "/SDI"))
 (segment (start 122.52 106.16) (end 122.52 104.77) (width 0.2) (layer "B.Cu") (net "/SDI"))
 (segment (start 116.52 121.74) (end 134.78 140) (width 0.2) (layer "B.Cu") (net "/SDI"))
 (segment (start 122.32 108.7) (end 117.52 113.5) (width 0.2) (layer "B.Cu") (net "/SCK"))
 (segment (start 117.52 120.2) (end 137.32 140) (width 0.2) (layer "B.Cu") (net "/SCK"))
 (segment (start 122.52 108.7) (end 122.32 108.7) (width 0.2) (layer "B.Cu") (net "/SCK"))
 (segment (start 117.52 113.5) (end 117.52 120.2) (width 0.2) (layer "B.Cu") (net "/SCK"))
 (segment (start 122.52 111.24) (end 120.78 111.24) (width 0.2) (layer "B.Cu") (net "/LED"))
 (segment (start 118.52 118.66) (end 139.86 140) (width 0.2) (layer "B.Cu") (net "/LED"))
 (segment (start 120.78 111.24) (end 118.52 113.5) (width 0.2) (layer "B.Cu") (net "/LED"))
 (segment (start 118.52 113.5) (end 118.52 118.66) (width 0.2) (layer "B.Cu") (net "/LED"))
 (segment (start 139.32967 136.92967) (end 142.4 140) (width 0.2) (layer "B.Cu") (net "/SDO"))
 (segment (start 139.32967 97.56967) (end 139.32967 136.92967) (width 0.2) (layer "B.Cu") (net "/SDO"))
 (segment (start 122.52 80.76) (end 139.32967 97.56967) (width 0.2) (layer "B.Cu") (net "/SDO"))
 (segment (start 141.44 136.5) (end 144.94 140) (width 0.2) (layer "B.Cu") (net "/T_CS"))
 (segment (start 141.02 96.72) (end 141.02 136.5) (width 0.2) (layer "B.Cu") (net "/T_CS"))
 (segment (start 141.02 136.5) (end 141.44 136.5) (width 0.2) (layer "B.Cu") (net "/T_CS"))
 (segment (start 122.52 78.22) (end 141.02 96.72) (width 0.2) (layer "B.Cu") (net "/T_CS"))
 (segment (start 143.02 135.54) (end 147.48 140) (width 0.2) (layer "B.Cu") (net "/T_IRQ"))
 (segment (start 143.02 96.18) (end 143.02 135.54) (width 0.2) (layer "B.Cu") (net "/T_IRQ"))
 (segment (start 122.52 75.68) (end 143.02 96.18) (width 0.2) (layer "B.Cu") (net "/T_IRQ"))
 (segment (start 113.34 61.42) (end 99.02 61.42) (width 0.2) (layer "F.Cu") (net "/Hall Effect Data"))
 (segment (start 122.52 70.6) (end 113.34 61.42) (width 0.2) (layer "F.Cu") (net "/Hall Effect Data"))
 (segment (start 140.52 60.5) (end 140.52 65.3) (width 0.2) (layer "F.Cu") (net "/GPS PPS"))
 (segment (start 172.06 53.5) (end 147.52 53.5) (width 0.2) (layer "F.Cu") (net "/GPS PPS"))
 (segment (start 147.52 53.5) (end 140.52 60.5) (width 0.2) (layer "F.Cu") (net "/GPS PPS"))
 (segment (start 140.52 65.3) (end 122.52 83.3) (width 0.2) (layer "F.Cu") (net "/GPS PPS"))
 (segment (start 175.56 57) (end 172.06 53.5) (width 0.2) (layer "F.Cu") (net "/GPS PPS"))
 (segment (start 122.52 85.84) (end 142.36 66) (width 0.2) (layer "F.Cu") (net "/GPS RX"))
 (segment (start 170.52 54.5) (end 173.02 57) (width 0.2) (layer "F.Cu") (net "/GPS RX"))
 (segment (start 142.52 60.5) (end 148.52 54.5) (width 0.2) (layer "F.Cu") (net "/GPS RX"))
 (segment (start 142.52 66) (end 142.52 60.5) (width 0.2) (layer "F.Cu") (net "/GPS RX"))
 (segment (start 148.52 54.5) (end 170.52 54.5) (width 0.2) (layer "F.Cu") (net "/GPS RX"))
 (segment (start 142.36 66) (end 142.52 66) (width 0.2) (layer "F.Cu") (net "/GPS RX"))
 (segment (start 144.02 66.88) (end 144.02 61) (width 0.2) (layer "F.Cu") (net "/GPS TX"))
 (segment (start 149.52 55.5) (end 168.98 55.5) (width 0.2) (layer "F.Cu") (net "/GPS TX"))
 (segment (start 144.02 61) (end 149.52 55.5) (width 0.2) (layer "F.Cu") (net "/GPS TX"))
 (segment (start 122.52 88.38) (end 144.02 66.88) (width 0.2) (layer "F.Cu") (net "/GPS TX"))
 (segment (start 168.98 55.5) (end 170.48 57) (width 0.2) (layer "F.Cu") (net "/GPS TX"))
 (segment (start 99.02 72.5) (end 102.02 75.5) (width 0.6) (layer "F.Cu") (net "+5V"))
 (segment (start 102.02 93.5) (end 102.24 93.5) (width 0.2) (layer "F.Cu") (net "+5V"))
 (segment (start 102.02 75.5) (end 102.02 93.5) (width 0.6) (layer "F.Cu") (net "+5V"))
 (segment (start 102.24 93.5) (end 122.52 113.78) (width 0.6) (layer "F.Cu") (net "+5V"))
 (segment (start 174.62 68.9) (end 174.52 69) (width 2) (layer "F.Cu") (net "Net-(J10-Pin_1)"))
 (segment (start 179.02 73.5) (end 190.02 73.5) (width 2) (layer "F.Cu") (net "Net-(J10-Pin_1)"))
 (segment (start 174.62 63.3425) (end 174.62 68.9) (width 2) (layer "F.Cu") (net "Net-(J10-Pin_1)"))
 (segment (start 174.52 69) (end 179.02 73.5) (width 2) (layer "F.Cu") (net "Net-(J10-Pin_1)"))
 (segment (start 190.0175 63.3425) (end 190.02 63.34) (width 0.2) (layer "F.Cu") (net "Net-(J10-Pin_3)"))
 (segment (start 179.62 63.3425) (end 190.0175 63.3425) (width 2) (layer "F.Cu") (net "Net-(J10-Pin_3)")))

